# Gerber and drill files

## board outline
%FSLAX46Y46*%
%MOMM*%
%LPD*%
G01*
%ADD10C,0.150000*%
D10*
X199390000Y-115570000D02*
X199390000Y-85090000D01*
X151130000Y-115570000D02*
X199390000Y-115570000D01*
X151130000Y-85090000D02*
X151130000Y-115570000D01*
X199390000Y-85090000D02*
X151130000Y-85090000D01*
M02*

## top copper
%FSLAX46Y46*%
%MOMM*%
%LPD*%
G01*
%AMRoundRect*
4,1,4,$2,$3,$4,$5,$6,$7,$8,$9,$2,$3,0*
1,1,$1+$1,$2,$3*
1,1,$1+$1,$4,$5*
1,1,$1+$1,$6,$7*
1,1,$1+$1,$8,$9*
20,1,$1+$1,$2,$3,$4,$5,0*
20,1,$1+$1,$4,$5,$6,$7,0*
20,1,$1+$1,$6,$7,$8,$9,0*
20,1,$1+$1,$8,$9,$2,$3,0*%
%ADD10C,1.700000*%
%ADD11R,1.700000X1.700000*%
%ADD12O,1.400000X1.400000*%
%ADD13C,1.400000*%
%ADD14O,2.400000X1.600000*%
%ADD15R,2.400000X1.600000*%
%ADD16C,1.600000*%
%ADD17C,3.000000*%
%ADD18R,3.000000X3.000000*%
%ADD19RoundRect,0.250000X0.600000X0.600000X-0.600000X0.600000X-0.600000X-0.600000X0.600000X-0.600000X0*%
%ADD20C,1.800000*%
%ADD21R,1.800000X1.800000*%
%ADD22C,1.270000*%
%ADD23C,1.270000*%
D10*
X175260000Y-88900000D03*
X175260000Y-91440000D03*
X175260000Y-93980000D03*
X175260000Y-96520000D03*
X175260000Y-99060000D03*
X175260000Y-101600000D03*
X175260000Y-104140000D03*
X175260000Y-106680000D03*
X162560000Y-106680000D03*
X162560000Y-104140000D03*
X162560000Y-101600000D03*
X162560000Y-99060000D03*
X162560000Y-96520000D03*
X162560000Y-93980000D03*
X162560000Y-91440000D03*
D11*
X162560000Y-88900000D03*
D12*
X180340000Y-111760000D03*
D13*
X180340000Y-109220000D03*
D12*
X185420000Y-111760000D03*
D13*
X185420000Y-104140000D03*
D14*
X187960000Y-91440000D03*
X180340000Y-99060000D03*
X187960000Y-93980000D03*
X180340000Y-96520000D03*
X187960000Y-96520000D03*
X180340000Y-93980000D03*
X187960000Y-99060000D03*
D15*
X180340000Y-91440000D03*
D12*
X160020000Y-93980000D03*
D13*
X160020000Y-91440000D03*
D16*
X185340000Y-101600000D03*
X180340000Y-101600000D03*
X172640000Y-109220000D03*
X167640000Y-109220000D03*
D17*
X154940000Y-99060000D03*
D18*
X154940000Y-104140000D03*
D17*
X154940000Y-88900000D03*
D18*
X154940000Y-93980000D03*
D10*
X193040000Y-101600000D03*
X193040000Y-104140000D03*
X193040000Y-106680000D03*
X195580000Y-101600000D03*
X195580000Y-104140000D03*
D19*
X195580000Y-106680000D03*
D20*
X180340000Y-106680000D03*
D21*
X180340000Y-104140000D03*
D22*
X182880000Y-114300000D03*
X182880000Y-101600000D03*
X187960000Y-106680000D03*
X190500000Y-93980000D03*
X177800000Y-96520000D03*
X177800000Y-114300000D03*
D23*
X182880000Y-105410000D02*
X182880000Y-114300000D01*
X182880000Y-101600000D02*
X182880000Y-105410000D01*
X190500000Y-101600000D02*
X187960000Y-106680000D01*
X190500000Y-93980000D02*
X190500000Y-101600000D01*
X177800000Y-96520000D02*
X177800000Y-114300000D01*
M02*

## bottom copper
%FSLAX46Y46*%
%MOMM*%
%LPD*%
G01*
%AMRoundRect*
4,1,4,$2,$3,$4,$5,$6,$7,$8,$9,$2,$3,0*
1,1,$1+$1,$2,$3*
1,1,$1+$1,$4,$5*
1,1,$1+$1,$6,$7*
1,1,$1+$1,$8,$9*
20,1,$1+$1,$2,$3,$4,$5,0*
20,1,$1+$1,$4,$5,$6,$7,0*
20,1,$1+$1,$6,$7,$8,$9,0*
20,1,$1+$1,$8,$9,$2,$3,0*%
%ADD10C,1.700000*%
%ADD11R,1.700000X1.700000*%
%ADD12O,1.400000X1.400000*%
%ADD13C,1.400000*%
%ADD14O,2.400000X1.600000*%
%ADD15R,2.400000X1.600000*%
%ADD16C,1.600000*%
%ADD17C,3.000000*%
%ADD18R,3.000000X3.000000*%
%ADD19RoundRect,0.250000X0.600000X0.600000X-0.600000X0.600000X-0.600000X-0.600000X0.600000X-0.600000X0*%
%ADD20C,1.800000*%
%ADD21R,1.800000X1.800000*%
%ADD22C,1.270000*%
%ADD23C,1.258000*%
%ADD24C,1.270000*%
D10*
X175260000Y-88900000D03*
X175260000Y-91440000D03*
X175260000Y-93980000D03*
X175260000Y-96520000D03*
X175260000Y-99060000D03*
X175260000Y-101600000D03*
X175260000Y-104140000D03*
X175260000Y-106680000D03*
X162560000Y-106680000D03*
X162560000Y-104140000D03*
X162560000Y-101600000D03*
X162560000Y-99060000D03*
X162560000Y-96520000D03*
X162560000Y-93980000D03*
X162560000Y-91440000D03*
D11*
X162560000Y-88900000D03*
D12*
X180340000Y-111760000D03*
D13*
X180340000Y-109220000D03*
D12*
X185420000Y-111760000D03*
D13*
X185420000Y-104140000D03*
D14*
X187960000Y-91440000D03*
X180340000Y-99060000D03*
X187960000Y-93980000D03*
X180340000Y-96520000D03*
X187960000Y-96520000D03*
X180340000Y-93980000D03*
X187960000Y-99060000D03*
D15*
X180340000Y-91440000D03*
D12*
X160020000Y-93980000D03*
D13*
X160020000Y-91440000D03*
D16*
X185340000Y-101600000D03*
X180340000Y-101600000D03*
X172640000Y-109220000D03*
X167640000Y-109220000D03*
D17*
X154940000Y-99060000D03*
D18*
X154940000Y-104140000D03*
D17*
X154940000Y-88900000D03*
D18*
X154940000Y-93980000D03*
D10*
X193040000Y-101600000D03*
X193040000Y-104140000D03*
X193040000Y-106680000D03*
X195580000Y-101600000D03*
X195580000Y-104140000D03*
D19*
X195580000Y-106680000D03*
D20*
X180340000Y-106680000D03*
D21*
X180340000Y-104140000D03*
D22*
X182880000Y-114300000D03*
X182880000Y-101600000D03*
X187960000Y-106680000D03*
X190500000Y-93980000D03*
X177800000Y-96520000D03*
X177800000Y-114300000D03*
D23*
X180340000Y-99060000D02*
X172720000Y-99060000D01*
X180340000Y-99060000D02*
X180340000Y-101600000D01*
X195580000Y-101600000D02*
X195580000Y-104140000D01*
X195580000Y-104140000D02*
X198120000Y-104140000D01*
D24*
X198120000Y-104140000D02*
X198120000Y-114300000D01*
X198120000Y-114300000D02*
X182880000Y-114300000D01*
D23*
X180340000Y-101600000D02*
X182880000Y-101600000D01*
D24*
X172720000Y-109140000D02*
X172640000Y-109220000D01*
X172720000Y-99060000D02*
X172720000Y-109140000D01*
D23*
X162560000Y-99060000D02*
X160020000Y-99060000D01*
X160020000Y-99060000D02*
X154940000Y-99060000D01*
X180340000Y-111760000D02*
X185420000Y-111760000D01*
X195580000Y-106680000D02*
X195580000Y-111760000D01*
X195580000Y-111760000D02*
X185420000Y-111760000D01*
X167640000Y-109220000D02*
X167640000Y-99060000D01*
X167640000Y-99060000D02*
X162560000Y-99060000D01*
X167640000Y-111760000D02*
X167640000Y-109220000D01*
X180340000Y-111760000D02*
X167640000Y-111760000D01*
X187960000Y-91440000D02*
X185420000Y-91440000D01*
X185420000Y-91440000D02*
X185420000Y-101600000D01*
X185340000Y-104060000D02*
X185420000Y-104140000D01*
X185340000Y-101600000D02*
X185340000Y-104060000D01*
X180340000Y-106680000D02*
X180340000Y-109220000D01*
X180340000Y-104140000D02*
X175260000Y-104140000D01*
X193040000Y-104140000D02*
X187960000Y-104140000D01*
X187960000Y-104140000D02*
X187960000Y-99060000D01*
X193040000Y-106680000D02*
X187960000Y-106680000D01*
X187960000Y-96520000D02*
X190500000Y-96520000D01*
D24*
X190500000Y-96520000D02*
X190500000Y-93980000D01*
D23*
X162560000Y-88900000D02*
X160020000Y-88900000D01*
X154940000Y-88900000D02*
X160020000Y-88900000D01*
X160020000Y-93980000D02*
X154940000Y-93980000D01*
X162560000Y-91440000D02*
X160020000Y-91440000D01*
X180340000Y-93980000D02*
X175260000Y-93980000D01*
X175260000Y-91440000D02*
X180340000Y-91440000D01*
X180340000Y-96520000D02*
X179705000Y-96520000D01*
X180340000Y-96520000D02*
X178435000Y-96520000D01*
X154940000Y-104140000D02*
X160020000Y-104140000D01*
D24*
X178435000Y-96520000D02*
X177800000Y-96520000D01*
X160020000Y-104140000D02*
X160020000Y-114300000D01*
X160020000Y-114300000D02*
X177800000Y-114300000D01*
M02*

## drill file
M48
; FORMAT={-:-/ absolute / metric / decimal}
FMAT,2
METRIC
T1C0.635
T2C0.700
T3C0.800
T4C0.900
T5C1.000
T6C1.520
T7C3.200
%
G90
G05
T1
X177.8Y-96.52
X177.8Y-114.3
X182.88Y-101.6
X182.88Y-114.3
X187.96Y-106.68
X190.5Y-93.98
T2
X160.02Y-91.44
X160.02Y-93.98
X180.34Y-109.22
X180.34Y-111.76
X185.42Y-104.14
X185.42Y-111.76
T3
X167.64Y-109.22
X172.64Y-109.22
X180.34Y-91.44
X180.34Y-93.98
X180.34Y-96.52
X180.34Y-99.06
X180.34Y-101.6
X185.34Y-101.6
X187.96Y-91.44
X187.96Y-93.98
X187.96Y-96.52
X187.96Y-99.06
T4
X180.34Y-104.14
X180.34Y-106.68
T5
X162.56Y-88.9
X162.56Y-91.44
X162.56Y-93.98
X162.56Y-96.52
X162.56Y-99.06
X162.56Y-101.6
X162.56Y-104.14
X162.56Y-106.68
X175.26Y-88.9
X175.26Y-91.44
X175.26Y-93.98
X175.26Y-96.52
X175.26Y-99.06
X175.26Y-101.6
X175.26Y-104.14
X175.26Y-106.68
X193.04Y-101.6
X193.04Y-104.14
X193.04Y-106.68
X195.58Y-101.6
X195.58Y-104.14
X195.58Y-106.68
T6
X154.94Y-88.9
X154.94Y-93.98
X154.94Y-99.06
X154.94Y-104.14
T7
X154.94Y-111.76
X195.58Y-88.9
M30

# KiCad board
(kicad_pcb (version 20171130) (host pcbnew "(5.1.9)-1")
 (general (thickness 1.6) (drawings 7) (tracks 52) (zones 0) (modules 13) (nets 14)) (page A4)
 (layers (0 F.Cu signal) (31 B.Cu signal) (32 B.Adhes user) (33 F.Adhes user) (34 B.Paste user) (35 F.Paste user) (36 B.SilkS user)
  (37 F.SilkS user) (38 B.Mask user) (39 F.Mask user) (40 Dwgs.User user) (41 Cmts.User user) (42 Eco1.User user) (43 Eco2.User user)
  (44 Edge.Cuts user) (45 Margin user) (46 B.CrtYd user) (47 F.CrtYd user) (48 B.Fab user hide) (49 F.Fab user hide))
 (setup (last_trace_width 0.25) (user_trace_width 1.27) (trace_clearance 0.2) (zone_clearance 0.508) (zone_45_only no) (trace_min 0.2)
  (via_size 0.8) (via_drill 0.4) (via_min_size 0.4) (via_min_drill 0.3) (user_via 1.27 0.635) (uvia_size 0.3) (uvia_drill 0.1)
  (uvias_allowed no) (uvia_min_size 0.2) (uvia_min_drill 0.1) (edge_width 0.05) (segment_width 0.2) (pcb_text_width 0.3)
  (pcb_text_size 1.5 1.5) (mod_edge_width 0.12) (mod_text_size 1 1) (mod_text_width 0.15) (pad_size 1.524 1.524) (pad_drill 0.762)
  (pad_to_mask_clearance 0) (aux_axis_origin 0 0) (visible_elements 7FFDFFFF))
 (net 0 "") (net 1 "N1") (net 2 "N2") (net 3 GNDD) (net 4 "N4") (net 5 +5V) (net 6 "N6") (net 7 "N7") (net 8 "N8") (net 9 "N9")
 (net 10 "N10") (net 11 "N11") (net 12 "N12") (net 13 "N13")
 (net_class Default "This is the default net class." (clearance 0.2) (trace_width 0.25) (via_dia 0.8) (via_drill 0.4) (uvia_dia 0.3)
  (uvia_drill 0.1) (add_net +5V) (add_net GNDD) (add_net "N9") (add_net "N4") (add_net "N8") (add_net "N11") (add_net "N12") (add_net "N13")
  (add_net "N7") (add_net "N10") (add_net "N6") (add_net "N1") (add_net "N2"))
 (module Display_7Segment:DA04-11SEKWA (layer F.Cu) (at 162.56 88.9)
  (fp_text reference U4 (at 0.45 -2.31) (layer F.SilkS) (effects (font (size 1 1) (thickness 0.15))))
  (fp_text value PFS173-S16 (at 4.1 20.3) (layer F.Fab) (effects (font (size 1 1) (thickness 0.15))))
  (pad 16 thru_hole circle (at 12.7 0) (size 1.7 1.7) (drill 1) (layers *.Cu *.Mask))
  (pad 15 thru_hole circle (at 12.7 2.54) (size 1.7 1.7) (drill 1) (layers *.Cu *.Mask) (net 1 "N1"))
  (pad 14 thru_hole circle (at 12.7 5.08) (size 1.7 1.7) (drill 1) (layers *.Cu *.Mask) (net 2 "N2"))
  (pad 13 thru_hole circle (at 12.7 7.62) (size 1.7 1.7) (drill 1) (layers *.Cu *.Mask))
  (pad 12 thru_hole circle (at 12.7 10.16) (size 1.7 1.7) (drill 1) (layers *.Cu *.Mask) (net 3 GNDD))
  (pad 11 thru_hole circle (at 12.7 12.7) (size 1.7 1.7) (drill 1) (layers *.Cu *.Mask))
  (pad 10 thru_hole circle (at 12.7 15.24) (size 1.7 1.7) (drill 1) (layers *.Cu *.Mask) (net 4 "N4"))
  (pad 9 thru_hole circle (at 12.7 17.78) (size 1.7 1.7) (drill 1) (layers *.Cu *.Mask))
  (pad 8 thru_hole circle (at 0 17.78) (size 1.7 1.7) (drill 1) (layers *.Cu *.Mask))
  (pad 7 thru_hole circle (at 0 15.24) (size 1.7 1.7) (drill 1) (layers *.Cu *.Mask))
  (pad 6 thru_hole circle (at 0 12.7) (size 1.7 1.7) (drill 1) (layers *.Cu *.Mask))
  (pad 5 thru_hole circle (at 0 10.16) (size 1.7 1.7) (drill 1) (layers *.Cu *.Mask) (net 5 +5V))
  (pad 4 thru_hole circle (at 0 7.62) (size 1.7 1.7) (drill 1) (layers *.Cu *.Mask))
  (pad 3 thru_hole circle (at 0 5.08) (size 1.7 1.7) (drill 1) (layers *.Cu *.Mask))
  (pad 2 thru_hole circle (at 0 2.54) (size 1.7 1.7) (drill 1) (layers *.Cu *.Mask) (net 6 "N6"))
  (pad 1 thru_hole rect (at 0 0) (size 1.7 1.7) (drill 1) (layers *.Cu *.Mask) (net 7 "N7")))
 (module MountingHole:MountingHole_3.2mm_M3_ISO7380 (layer F.Cu) (at 154.94 111.76)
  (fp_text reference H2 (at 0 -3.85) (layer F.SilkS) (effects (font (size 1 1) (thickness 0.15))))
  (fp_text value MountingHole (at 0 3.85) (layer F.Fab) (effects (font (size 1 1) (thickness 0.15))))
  (pad 1 np_thru_hole circle (at 0 0) (size 3.2 3.2) (drill 3.2) (layers *.Cu *.Mask)))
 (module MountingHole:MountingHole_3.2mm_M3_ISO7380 (layer F.Cu) (at 195.58 88.9)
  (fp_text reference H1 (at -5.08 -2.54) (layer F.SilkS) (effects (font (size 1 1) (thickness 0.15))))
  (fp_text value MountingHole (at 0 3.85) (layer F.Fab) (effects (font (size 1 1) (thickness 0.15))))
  (pad 1 np_thru_hole circle (at 0 0) (size 3.2 3.2) (drill 3.2) (layers *.Cu *.Mask)))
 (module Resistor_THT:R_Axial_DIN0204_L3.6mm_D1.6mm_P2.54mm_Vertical (layer F.Cu) (at 180.34 109.22 270)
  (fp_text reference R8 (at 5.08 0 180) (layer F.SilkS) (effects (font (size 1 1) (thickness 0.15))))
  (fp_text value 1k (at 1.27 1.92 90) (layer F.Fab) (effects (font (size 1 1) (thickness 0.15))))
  (pad 2 thru_hole oval (at 2.54 0 270) (size 1.4 1.4) (drill 0.7) (layers *.Cu *.Mask) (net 5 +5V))
  (pad 1 thru_hole circle (at 0 0 270) (size 1.4 1.4) (drill 0.7) (layers *.Cu *.Mask) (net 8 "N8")))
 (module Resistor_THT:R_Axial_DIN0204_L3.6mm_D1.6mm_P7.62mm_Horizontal (layer F.Cu) (at 185.42 104.14 270)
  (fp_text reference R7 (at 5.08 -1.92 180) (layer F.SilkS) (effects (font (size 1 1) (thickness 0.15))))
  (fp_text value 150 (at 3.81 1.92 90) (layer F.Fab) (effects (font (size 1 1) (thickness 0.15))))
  (pad 2 thru_hole oval (at 7.62 0 270) (size 1.4 1.4) (drill 0.7) (layers *.Cu *.Mask) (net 5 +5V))
  (pad 1 thru_hole circle (at 0 0 270) (size 1.4 1.4) (drill 0.7) (layers *.Cu *.Mask) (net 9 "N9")))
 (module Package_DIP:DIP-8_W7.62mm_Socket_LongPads (layer F.Cu) (at 180.34 91.44)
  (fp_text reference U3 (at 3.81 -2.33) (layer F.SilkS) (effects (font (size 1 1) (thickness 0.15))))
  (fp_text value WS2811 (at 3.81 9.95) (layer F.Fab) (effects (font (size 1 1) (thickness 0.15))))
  (pad 8 thru_hole oval (at 7.62 0) (size 2.4 1.6) (drill 0.8) (layers *.Cu *.Mask) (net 9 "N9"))
  (pad 4 thru_hole oval (at 0 7.62) (size 2.4 1.6) (drill 0.8) (layers *.Cu *.Mask) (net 3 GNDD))
  (pad 7 thru_hole oval (at 7.62 2.54) (size 2.4 1.6) (drill 0.8) (layers *.Cu *.Mask))
  (pad 3 thru_hole oval (at 0 5.08) (size 2.4 1.6) (drill 0.8) (layers *.Cu *.Mask) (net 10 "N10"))
  (pad 6 thru_hole oval (at 7.62 5.08) (size 2.4 1.6) (drill 0.8) (layers *.Cu *.Mask) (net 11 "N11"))
  (pad 2 thru_hole oval (at 0 2.54) (size 2.4 1.6) (drill 0.8) (layers *.Cu *.Mask) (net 2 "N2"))
  (pad 5 thru_hole oval (at 7.62 7.62) (size 2.4 1.6) (drill 0.8) (layers *.Cu *.Mask) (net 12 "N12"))
  (pad 1 thru_hole rect (at 0 0) (size 2.4 1.6) (drill 0.8) (layers *.Cu *.Mask) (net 1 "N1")))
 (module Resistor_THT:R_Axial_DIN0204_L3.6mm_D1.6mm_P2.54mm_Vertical (layer F.Cu) (at 160.02 91.44 270)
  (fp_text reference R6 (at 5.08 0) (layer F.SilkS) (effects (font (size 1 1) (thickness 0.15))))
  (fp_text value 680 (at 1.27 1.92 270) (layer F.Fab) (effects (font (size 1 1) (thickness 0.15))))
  (pad 2 thru_hole oval (at 2.54 0 270) (size 1.4 1.4) (drill 0.7) (layers *.Cu *.Mask) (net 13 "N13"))
  (pad 1 thru_hole circle (at 0 0 270) (size 1.4 1.4) (drill 0.7) (layers *.Cu *.Mask) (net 6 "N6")))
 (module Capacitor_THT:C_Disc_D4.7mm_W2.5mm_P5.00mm (layer F.Cu) (at 180.34 101.6)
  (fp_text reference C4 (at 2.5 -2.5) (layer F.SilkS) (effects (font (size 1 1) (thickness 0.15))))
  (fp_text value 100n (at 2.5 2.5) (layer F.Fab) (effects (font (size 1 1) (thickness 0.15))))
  (pad 2 thru_hole circle (at 5 0) (size 1.6 1.6) (drill 0.8) (layers *.Cu *.Mask) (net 9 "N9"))
  (pad 1 thru_hole circle (at 0 0) (size 1.6 1.6) (drill 0.8) (layers *.Cu *.Mask) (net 3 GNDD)))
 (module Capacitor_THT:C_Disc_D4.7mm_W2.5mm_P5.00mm (layer F.Cu) (at 167.64 109.22)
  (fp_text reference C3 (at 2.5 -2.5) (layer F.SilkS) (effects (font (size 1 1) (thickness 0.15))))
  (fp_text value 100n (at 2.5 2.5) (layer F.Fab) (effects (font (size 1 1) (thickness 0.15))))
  (pad 2 thru_hole circle (at 5 0) (size 1.6 1.6) (drill 0.8) (layers *.Cu *.Mask) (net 3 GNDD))
  (pad 1 thru_hole circle (at 0 0) (size 1.6 1.6) (drill 0.8) (layers *.Cu *.Mask) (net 5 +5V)))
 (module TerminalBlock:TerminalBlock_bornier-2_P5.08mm (layer F.Cu) (at 154.94 104.14 90)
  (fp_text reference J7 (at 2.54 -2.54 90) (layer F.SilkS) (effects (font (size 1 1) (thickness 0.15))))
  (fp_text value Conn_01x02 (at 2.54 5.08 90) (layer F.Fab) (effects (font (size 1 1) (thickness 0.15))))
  (pad 2 thru_hole circle (at 5.08 0 90) (size 3 3) (drill 1.52) (layers *.Cu *.Mask) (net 5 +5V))
  (pad 1 thru_hole rect (at 0 0 90) (size 3 3) (drill 1.52) (layers *.Cu *.Mask) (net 10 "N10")))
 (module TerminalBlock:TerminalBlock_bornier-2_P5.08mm (layer F.Cu) (at 154.94 93.98 90)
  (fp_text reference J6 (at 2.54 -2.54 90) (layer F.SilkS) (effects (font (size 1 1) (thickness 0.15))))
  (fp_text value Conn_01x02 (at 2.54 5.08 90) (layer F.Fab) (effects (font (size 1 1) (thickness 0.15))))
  (pad 2 thru_hole circle (at 5.08 0 90) (size 3 3) (drill 1.52) (layers *.Cu *.Mask) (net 7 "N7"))
  (pad 1 thru_hole rect (at 0 0 90) (size 3 3) (drill 1.52) (layers *.Cu *.Mask) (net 13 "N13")))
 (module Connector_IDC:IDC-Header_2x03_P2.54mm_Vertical (layer F.Cu) (at 195.58 106.68 180)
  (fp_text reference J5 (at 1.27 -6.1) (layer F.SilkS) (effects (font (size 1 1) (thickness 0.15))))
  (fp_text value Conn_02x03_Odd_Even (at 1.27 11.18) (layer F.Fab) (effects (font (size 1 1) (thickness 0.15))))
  (pad 6 thru_hole circle (at 2.54 5.08 180) (size 1.7 1.7) (drill 1) (layers *.Cu *.Mask))
  (pad 4 thru_hole circle (at 2.54 2.54 180) (size 1.7 1.7) (drill 1) (layers *.Cu *.Mask) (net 12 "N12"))
  (pad 2 thru_hole circle (at 2.54 0 180) (size 1.7 1.7) (drill 1) (layers *.Cu *.Mask) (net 11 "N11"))
  (pad 5 thru_hole circle (at 0 5.08 180) (size 1.7 1.7) (drill 1) (layers *.Cu *.Mask) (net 3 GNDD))
  (pad 3 thru_hole circle (at 0 2.54 180) (size 1.7 1.7) (drill 1) (layers *.Cu *.Mask) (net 3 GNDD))
  (pad 1 thru_hole roundrect (at 0 0 180) (size 1.7 1.7) (drill 1) (layers *.Cu *.Mask) (roundrect_rratio 0.1470588235294118) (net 5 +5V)))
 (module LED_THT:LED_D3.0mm (layer F.Cu) (at 180.34 104.14 270)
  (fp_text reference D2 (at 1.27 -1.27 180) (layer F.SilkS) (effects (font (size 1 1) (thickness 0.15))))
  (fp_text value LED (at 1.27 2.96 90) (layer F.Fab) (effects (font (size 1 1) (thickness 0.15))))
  (pad 2 thru_hole circle (at 2.54 0 270) (size 1.8 1.8) (drill 0.9) (layers *.Cu *.Mask) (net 8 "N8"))
  (pad 1 thru_hole rect (at 0 0 270) (size 1.8 1.8) (drill 0.9) (layers *.Cu *.Mask) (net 4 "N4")))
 (gr_line (start 199.39 115.57) (end 199.39 85.09) (layer Edge.Cuts) (width 0.15))
 (gr_line (start 151.13 115.57) (end 199.39 115.57) (layer Edge.Cuts) (width 0.15))
 (gr_line (start 151.13 85.09) (end 151.13 115.57) (layer Edge.Cuts) (width 0.15))
 (gr_line (start 199.39 85.09) (end 151.13 85.09) (layer Edge.Cuts) (width 0.15))
 (segment (start 180.34 99.06) (end 172.72 99.06) (width 1.258) (layer B.Cu) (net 3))
 (segment (start 180.34 99.06) (end 180.34 101.6) (width 1.258) (layer B.Cu) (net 3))
 (segment (start 195.58 101.6) (end 195.58 104.14) (width 1.258) (layer B.Cu) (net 3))
 (segment (start 195.58 104.14) (end 198.12 104.14) (width 1.258) (layer B.Cu) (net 3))
 (segment (start 198.12 104.14) (end 198.12 114.3) (width 1.27) (layer B.Cu) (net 3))
 (segment (start 198.12 114.3) (end 182.88 114.3) (width 1.27) (layer B.Cu) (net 3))
 (via (at 182.88 114.3) (size 1.27) (drill 0.635) (layers F.Cu B.Cu) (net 3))
 (segment (start 182.88 105.41) (end 182.88 114.3) (width 1.27) (layer F.Cu) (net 3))
 (segment (start 182.88 101.6) (end 182.88 105.41) (width 1.27) (layer F.Cu) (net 3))
 (via (at 182.88 101.6) (size 1.27) (drill 0.635) (layers F.Cu B.Cu) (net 3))
 (segment (start 180.34 101.6) (end 182.88 101.6) (width 1.258) (layer B.Cu) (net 3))
 (segment (start 172.72 109.14) (end 172.64 109.22) (width 1.27) (layer B.Cu) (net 3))
 (segment (start 172.72 99.06) (end 172.72 109.14) (width 1.27) (layer B.Cu) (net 3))
 (segment (start 162.56 99.06) (end 160.02 99.06) (width 1.258) (layer B.Cu) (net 5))
 (segment (start 160.02 99.06) (end 154.94 99.06) (width 1.258) (layer B.Cu) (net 5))
 (segment (start 180.34 111.76) (end 185.42 111.76) (width 1.258) (layer B.Cu) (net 5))
 (segment (start 195.58 106.68) (end 195.58 111.76) (width 1.258) (layer B.Cu) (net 5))
 (segment (start 195.58 111.76) (end 185.42 111.76) (width 1.258) (layer B.Cu) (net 5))
 (segment (start 167.64 109.22) (end 167.64 99.06) (width 1.258) (layer B.Cu) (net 5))
 (segment (start 167.64 99.06) (end 162.56 99.06) (width 1.258) (layer B.Cu) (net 5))
 (segment (start 167.64 111.76) (end 167.64 109.22) (width 1.258) (layer B.Cu) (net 5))
 (segment (start 180.34 111.76) (end 167.64 111.76) (width 1.258) (layer B.Cu) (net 5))
 (segment (start 187.96 91.44) (end 185.42 91.44) (width 1.258) (layer B.Cu) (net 9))
 (segment (start 185.42 91.44) (end 185.42 101.6) (width 1.258) (layer B.Cu) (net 9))
 (segment (start 185.34 104.06) (end 185.42 104.14) (width 1.258) (layer B.Cu) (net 9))
 (segment (start 185.34 101.6) (end 185.34 104.06) (width 1.258) (layer B.Cu) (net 9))
 (segment (start 180.34 106.68) (end 180.34 109.22) (width 1.258) (layer B.Cu) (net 8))
 (segment (start 180.34 104.14) (end 175.26 104.14) (width 1.258) (layer B.Cu) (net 4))
 (segment (start 193.04 104.14) (end 187.96 104.14) (width 1.258) (layer B.Cu) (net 12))
 (segment (start 187.96 104.14) (end 187.96 99.06) (width 1.258) (layer B.Cu) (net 12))
 (segment (start 193.04 106.68) (end 187.96 106.68) (width 1.258) (layer B.Cu) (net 11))
 (via (at 187.96 106.68) (size 1.27) (drill 0.635) (layers F.Cu B.Cu) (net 11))
 (segment (start 187.96 96.52) (end 190.5 96.52) (width 1.258) (layer B.Cu) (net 11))
 (segment (start 190.5 101.6) (end 187.96 106.68) (width 1.27) (layer F.Cu) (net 11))
 (segment (start 190.5 93.98) (end 190.5 101.6) (width 1.27) (layer F.Cu) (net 11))
 (via (at 190.5 93.98) (size 1.27) (drill 0.635) (layers F.Cu B.Cu) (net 11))
 (segment (start 190.5 96.52) (end 190.5 93.98) (width 1.27) (layer B.Cu) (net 11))
 (segment (start 162.56 88.9) (end 160.02 88.9) (width 1.258) (layer B.Cu) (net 7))
 (segment (start 154.94 88.9) (end 160.02 88.9) (width 1.258) (layer B.Cu) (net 7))
 (segment (start 160.02 93.98) (end 154.94 93.98) (width 1.258) (layer B.Cu) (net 13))
 (segment (start 162.56 91.44) (end 160.02 91.44) (width 1.258) (layer B.Cu) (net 6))
 (segment (start 180.34 93.98) (end 175.26 93.98) (width 1.258) (layer B.Cu) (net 2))
 (segment (start 175.26 91.44) (end 180.34 91.44) (width 1.258) (layer B.Cu) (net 1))
 (segment (start 180.34 96.52) (end 179.705 96.52) (width 1.258) (layer B.Cu) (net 10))
 (segment (start 180.34 96.52) (end 178.435 96.52) (width 1.258) (layer B.Cu) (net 10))
 (segment (start 154.94 104.14) (end 160.02 104.14) (width 1.258) (layer B.Cu) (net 10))
 (segment (start 178.435 96.52) (end 177.8 96.52) (width 1.27) (layer B.Cu) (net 10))
 (via (at 177.8 96.52) (size 1.27) (drill 0.635) (layers F.Cu B.Cu) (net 10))
 (segment (start 177.8 96.52) (end 177.8 114.3) (width 1.27) (layer F.Cu) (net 10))
 (segment (start 160.02 104.14) (end 160.02 114.3) (width 1.27) (layer B.Cu) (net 10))
 (segment (start 160.02 114.3) (end 177.8 114.3) (width 1.27) (layer B.Cu) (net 10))
 (via (at 177.8 114.3) (size 1.27) (drill 0.635) (layers F.Cu B.Cu) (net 10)))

